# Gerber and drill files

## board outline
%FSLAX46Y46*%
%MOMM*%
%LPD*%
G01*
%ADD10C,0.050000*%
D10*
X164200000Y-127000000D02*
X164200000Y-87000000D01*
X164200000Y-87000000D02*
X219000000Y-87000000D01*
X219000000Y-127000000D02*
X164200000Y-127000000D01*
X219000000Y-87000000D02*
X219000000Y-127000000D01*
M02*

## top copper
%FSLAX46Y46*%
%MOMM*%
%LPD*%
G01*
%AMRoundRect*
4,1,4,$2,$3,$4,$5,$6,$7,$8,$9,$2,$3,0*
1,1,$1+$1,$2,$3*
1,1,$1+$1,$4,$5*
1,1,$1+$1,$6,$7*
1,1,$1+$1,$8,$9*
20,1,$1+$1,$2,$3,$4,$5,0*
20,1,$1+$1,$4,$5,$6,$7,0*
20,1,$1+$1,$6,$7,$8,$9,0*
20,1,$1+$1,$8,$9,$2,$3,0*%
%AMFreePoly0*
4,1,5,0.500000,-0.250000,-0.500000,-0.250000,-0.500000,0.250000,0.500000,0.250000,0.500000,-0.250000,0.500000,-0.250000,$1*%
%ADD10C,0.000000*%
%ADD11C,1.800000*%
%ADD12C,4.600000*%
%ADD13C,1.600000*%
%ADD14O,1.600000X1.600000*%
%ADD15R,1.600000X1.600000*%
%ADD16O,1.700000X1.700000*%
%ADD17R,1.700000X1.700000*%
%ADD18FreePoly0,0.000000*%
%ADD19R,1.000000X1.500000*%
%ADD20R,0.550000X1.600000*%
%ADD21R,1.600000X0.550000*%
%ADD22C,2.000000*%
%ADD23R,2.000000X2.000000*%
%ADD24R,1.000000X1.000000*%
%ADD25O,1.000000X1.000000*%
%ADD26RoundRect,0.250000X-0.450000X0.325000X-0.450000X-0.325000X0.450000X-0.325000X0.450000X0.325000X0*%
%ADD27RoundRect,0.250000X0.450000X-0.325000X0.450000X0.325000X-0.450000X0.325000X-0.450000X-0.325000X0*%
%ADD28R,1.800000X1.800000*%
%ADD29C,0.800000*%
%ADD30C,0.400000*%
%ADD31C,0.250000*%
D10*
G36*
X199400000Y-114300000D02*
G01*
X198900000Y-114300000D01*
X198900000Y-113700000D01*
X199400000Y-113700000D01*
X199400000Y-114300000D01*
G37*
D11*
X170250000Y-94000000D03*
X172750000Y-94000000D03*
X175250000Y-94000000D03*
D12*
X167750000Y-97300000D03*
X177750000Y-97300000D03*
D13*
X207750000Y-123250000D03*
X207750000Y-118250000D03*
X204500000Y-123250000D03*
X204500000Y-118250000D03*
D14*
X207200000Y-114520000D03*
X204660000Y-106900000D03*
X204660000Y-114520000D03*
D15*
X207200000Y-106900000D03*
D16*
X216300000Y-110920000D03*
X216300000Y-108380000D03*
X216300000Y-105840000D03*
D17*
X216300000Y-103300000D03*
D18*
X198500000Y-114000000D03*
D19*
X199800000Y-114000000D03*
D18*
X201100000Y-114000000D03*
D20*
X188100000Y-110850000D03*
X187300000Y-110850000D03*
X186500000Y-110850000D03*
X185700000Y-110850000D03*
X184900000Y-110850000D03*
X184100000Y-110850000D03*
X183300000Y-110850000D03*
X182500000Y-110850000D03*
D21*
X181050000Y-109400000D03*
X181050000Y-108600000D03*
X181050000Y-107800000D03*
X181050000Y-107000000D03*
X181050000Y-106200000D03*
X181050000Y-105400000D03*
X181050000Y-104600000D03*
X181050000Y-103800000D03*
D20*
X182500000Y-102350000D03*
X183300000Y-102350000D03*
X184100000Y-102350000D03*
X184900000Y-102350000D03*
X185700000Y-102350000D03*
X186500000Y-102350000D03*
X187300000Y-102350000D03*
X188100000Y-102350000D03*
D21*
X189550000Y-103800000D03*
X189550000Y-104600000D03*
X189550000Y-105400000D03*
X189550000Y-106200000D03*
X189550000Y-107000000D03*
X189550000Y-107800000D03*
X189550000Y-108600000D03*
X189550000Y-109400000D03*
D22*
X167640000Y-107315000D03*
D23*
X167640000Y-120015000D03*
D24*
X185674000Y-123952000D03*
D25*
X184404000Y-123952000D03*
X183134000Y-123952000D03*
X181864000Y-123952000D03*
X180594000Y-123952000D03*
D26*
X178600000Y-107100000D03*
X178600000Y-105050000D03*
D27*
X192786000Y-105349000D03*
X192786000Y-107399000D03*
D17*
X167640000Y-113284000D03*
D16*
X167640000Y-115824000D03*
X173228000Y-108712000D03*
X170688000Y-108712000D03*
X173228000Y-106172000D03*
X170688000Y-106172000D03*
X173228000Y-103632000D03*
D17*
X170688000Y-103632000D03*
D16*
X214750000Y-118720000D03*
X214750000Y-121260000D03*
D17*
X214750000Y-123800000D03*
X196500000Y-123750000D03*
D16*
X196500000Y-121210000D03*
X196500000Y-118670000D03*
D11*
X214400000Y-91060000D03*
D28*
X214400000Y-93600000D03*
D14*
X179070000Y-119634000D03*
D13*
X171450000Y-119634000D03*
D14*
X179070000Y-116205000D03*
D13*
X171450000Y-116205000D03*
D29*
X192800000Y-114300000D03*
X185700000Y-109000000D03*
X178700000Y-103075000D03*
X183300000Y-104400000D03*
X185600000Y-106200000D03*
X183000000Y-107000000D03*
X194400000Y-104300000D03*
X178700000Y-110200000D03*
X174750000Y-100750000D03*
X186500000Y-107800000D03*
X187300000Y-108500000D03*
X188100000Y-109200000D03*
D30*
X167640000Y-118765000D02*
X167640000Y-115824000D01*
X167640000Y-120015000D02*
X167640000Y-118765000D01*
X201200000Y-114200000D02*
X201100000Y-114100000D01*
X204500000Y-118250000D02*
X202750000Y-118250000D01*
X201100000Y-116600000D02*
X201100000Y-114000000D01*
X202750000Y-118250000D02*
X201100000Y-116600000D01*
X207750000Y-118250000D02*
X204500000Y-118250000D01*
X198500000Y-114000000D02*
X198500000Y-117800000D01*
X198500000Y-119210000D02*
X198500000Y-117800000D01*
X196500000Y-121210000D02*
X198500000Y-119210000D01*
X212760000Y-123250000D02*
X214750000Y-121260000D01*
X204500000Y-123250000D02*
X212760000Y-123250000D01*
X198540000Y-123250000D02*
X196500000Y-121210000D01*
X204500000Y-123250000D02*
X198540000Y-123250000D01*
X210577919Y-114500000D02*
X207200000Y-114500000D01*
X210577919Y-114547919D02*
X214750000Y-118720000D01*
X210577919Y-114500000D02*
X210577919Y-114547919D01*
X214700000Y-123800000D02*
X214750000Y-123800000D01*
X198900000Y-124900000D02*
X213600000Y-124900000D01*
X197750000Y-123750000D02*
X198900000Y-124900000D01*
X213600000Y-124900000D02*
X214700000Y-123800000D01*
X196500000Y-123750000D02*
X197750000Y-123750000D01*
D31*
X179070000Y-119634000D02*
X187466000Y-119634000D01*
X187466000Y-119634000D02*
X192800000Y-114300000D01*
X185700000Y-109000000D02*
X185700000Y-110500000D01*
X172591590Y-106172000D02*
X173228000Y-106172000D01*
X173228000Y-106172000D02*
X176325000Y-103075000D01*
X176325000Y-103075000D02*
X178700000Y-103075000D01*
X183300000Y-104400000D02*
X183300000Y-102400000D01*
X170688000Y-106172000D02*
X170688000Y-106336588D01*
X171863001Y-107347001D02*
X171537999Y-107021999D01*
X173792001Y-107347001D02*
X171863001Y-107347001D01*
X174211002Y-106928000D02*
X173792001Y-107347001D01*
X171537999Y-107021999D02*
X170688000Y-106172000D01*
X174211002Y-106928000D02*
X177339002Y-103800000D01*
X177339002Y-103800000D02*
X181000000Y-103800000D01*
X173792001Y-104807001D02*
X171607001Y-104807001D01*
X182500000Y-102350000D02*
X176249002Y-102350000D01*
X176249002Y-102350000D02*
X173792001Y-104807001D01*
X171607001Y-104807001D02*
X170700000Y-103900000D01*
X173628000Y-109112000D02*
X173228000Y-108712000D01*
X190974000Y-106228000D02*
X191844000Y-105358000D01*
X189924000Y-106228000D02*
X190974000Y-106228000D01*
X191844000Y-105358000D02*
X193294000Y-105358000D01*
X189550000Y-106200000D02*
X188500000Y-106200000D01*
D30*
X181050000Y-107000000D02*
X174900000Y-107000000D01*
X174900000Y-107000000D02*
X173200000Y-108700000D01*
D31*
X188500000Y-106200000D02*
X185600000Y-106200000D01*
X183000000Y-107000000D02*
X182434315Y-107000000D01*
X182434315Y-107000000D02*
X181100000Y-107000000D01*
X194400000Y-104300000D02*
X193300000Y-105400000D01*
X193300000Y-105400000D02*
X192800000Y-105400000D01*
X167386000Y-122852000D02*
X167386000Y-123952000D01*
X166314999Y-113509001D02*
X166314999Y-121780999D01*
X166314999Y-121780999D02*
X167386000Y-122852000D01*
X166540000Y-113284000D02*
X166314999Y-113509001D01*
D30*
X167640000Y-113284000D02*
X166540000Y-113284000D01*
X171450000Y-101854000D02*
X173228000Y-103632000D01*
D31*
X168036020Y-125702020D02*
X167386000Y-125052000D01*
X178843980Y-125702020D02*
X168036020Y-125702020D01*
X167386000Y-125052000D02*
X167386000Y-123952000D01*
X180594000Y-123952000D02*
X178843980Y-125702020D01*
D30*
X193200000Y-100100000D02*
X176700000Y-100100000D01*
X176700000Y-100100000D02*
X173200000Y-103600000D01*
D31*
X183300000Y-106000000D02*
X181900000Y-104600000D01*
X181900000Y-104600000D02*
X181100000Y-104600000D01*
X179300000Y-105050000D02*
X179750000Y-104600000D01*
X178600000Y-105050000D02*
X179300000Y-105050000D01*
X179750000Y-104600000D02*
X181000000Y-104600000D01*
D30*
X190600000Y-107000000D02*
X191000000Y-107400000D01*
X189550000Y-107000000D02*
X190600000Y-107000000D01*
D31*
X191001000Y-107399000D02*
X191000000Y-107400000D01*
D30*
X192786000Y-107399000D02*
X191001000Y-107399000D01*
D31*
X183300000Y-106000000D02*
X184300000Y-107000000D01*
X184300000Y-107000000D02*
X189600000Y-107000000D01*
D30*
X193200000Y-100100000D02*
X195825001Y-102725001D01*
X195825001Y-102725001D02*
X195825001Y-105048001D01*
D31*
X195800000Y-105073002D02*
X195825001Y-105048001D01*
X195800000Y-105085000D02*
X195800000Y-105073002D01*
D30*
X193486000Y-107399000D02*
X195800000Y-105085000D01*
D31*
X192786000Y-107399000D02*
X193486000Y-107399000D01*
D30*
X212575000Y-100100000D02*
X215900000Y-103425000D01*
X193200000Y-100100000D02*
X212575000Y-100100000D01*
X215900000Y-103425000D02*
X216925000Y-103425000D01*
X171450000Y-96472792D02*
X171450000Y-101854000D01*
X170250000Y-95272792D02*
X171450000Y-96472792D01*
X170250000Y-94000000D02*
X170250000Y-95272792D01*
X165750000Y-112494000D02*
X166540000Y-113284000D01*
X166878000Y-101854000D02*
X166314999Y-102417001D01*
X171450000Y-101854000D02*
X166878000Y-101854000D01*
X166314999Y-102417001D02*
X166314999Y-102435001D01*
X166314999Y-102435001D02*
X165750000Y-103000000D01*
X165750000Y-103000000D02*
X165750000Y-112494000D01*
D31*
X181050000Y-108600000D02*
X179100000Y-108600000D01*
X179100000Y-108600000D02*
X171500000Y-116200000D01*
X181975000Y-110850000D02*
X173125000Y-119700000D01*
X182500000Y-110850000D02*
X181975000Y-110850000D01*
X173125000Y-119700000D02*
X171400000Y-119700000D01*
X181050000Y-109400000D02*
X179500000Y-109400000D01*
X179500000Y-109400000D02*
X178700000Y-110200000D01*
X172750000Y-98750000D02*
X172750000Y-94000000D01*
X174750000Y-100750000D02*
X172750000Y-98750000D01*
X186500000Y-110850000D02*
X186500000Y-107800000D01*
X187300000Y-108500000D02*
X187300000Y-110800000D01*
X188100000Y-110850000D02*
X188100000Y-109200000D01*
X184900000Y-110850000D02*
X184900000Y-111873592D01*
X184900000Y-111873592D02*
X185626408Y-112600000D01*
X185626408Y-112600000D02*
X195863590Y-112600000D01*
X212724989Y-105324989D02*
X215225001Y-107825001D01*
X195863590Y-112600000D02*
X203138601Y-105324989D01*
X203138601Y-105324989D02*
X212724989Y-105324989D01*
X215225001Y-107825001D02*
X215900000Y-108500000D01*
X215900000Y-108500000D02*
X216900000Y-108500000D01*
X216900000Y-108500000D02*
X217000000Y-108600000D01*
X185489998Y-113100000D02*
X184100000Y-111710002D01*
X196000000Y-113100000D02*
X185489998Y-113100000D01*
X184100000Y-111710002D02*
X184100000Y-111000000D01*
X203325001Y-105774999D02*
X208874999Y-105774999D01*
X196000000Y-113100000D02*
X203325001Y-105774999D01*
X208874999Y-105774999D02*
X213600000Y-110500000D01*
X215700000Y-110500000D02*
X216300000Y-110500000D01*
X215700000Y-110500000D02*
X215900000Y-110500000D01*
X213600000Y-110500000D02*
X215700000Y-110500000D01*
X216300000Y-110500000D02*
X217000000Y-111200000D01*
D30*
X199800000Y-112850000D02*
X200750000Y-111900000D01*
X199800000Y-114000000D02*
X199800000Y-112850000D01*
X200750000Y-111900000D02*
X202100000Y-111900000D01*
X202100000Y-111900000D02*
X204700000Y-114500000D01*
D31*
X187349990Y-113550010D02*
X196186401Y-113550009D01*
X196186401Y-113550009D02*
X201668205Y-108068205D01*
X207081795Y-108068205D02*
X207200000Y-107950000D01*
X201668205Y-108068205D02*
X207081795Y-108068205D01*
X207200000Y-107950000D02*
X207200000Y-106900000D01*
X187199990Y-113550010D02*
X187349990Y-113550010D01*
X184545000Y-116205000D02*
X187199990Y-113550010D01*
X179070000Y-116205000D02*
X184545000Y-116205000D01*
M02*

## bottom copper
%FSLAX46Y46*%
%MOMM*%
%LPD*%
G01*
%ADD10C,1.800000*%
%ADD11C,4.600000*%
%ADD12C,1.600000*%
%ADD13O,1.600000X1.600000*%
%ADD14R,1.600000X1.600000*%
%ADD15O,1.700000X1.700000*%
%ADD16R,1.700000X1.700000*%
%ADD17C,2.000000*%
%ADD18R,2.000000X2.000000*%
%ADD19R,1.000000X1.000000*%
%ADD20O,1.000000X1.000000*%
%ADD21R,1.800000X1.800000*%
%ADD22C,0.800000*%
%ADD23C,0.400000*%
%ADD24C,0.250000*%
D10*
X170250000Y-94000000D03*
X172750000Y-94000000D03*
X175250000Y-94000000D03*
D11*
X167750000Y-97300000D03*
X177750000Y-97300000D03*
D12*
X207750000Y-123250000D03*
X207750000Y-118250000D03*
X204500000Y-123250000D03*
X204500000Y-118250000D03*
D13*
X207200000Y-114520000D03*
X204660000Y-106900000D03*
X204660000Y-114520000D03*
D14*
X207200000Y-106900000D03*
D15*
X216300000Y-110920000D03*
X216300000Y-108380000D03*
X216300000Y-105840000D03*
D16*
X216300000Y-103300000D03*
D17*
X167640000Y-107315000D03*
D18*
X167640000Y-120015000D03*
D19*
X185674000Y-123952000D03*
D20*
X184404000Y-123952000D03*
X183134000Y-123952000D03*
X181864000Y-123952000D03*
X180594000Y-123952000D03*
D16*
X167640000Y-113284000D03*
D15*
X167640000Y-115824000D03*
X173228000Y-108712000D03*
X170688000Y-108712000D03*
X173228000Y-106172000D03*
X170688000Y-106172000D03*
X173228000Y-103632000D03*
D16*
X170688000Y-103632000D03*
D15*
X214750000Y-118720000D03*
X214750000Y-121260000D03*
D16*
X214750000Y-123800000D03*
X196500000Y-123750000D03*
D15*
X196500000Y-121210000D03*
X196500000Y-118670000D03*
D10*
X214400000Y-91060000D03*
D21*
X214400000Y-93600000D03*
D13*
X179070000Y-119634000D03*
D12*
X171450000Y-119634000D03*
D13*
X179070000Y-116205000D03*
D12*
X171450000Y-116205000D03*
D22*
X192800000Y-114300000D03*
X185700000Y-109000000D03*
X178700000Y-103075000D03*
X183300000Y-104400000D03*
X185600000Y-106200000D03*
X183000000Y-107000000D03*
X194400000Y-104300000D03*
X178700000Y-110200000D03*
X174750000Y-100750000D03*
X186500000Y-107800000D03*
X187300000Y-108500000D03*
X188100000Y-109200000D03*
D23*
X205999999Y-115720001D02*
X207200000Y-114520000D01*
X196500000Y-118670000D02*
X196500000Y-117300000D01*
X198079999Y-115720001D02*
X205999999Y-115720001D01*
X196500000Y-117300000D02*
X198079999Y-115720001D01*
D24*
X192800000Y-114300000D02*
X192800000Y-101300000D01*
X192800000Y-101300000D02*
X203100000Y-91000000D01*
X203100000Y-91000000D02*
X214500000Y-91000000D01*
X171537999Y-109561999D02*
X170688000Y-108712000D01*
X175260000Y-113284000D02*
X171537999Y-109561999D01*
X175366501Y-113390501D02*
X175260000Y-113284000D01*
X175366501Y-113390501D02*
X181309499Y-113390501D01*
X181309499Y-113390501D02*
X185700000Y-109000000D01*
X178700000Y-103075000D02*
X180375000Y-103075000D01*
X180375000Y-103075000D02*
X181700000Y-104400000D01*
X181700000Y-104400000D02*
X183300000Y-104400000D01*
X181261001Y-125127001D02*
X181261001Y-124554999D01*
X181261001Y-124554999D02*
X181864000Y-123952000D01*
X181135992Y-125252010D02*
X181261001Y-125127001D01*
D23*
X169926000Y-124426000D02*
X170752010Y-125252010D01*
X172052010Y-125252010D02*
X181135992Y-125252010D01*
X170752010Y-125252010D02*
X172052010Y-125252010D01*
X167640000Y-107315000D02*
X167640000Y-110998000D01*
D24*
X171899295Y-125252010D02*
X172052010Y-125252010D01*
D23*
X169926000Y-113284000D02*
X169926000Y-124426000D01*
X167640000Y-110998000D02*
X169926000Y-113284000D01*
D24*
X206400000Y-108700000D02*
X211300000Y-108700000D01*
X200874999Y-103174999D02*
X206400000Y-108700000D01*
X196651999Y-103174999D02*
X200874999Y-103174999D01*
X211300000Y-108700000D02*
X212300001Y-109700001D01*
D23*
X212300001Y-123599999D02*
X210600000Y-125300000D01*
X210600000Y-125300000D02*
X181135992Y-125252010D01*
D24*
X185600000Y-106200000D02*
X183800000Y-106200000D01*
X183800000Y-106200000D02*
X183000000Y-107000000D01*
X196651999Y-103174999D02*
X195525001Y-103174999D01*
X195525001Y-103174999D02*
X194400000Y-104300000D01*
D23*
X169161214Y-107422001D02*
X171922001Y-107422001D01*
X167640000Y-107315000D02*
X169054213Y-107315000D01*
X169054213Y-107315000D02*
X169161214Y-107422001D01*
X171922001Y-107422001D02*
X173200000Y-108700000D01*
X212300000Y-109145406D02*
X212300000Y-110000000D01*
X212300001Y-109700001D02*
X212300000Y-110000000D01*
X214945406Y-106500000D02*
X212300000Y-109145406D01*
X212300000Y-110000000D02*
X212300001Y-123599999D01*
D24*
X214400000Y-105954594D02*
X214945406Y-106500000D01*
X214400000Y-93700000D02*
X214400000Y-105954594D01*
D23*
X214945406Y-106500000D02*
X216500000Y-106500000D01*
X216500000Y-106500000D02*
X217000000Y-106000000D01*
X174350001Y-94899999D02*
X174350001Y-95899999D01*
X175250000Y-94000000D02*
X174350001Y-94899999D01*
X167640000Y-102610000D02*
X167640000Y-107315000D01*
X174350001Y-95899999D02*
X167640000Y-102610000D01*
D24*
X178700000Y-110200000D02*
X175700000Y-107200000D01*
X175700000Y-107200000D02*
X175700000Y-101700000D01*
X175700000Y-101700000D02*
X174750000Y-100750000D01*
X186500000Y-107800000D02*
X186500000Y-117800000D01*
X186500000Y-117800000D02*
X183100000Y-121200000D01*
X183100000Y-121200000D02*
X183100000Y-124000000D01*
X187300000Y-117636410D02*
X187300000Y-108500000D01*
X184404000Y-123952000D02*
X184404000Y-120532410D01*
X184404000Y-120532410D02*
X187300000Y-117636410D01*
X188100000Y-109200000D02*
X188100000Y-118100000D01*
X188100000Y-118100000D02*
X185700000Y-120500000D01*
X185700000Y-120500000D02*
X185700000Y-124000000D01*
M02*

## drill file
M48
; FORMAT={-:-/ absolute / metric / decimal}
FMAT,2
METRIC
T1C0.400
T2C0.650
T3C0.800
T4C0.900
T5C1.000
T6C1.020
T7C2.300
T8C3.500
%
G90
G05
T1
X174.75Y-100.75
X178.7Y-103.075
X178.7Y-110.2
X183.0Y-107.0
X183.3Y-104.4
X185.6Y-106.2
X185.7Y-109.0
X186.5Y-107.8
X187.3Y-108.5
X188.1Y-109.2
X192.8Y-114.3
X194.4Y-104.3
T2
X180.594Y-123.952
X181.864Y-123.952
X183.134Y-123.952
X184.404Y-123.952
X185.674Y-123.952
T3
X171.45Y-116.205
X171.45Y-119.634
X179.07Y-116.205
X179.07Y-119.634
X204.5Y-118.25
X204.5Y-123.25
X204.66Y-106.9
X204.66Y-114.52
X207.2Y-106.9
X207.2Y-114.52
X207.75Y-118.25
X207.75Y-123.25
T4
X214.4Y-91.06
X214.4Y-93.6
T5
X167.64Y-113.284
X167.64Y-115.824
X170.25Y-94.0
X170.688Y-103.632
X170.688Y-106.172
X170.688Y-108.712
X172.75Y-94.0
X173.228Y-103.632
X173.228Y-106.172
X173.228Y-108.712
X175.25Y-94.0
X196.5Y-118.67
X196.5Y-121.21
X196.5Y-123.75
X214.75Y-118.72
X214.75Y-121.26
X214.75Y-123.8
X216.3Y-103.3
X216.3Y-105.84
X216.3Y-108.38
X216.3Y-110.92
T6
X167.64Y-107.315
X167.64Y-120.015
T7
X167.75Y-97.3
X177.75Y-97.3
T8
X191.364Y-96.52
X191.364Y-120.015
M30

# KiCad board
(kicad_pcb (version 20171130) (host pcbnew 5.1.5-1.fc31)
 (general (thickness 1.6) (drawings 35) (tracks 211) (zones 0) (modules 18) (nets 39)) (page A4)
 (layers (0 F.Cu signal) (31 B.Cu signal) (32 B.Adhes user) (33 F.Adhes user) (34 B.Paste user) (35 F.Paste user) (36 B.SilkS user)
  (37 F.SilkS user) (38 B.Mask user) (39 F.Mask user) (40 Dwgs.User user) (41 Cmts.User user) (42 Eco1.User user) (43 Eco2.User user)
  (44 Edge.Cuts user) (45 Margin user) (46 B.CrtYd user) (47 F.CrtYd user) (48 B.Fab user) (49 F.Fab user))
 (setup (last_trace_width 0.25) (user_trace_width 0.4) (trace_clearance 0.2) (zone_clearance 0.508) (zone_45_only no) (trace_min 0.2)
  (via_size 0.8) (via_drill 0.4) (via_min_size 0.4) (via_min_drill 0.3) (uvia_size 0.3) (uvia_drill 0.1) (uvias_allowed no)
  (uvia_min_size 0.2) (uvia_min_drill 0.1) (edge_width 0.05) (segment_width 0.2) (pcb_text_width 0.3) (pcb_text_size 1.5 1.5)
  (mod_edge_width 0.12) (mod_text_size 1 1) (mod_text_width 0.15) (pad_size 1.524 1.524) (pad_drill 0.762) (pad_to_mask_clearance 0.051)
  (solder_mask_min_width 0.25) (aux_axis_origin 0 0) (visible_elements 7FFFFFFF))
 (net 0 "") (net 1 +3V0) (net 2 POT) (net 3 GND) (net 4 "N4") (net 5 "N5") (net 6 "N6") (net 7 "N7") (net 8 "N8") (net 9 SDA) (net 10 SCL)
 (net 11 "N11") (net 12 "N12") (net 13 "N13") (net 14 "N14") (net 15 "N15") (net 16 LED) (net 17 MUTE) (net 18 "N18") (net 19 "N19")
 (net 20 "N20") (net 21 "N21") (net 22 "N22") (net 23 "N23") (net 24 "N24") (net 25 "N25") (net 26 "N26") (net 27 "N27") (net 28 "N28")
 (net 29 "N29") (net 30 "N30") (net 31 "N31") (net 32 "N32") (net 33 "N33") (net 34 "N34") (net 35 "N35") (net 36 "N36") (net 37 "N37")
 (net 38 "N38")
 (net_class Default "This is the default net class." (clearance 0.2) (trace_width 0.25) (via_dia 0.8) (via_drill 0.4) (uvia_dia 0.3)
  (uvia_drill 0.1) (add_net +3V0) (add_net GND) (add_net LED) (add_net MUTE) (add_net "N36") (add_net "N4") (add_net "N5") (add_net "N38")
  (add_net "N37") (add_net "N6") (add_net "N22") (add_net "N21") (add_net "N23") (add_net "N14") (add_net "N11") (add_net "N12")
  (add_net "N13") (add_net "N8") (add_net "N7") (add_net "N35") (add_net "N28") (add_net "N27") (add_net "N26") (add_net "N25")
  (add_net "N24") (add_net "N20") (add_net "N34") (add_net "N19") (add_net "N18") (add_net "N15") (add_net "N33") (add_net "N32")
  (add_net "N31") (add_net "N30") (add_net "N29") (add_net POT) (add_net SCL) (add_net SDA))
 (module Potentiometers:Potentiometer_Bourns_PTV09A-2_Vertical (layer F.Cu) (at 175.25 94 90)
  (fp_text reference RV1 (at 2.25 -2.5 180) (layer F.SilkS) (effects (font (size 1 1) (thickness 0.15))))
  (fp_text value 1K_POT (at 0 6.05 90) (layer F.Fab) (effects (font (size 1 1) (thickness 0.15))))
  (pad 3 thru_hole circle (at 0 -5 90) (size 1.8 1.8) (drill 1) (layers *.Cu *.Mask) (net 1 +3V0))
  (pad 2 thru_hole circle (at 0 -2.5 90) (size 1.8 1.8) (drill 1) (layers *.Cu *.Mask) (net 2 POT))
  (pad 1 thru_hole circle (at 0 0 90) (size 1.8 1.8) (drill 1) (layers *.Cu *.Mask) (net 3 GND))
  (pad 0 thru_hole circle (at -3.3 -7.5 90) (size 4.6 4.6) (drill 2.3) (layers *.Cu *.Mask))
  (pad 0 thru_hole circle (at -3.3 2.5 90) (size 4.6 4.6) (drill 2.3) (layers *.Cu *.Mask)))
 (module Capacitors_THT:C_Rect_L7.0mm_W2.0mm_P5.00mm (layer F.Cu) (at 207.75 123.25 90)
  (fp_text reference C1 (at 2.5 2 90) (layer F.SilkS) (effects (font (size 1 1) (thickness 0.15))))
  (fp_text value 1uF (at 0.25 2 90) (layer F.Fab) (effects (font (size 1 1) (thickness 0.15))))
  (pad 1 thru_hole circle (at 0 0 90) (size 1.6 1.6) (drill 0.8) (layers *.Cu *.Mask) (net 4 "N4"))
  (pad 2 thru_hole circle (at 5 0 90) (size 1.6 1.6) (drill 0.8) (layers *.Cu *.Mask) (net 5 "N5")))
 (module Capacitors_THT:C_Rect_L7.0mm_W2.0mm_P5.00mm (layer F.Cu) (at 204.5 123.25 90)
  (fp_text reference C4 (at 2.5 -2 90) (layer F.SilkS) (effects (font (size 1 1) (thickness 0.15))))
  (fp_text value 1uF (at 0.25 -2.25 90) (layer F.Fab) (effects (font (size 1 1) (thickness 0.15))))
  (pad 1 thru_hole circle (at 0 0 90) (size 1.6 1.6) (drill 0.8) (layers *.Cu *.Mask) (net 4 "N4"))
  (pad 2 thru_hole circle (at 5 0 90) (size 1.6 1.6) (drill 0.8) (layers *.Cu *.Mask) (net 5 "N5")))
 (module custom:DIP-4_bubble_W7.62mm (layer F.Cu) (at 207.2 106.9 270)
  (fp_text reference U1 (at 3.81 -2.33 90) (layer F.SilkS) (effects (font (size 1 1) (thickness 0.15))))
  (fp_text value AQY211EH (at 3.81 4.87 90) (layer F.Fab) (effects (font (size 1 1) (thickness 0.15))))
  (pad 4 thru_hole oval (at 7.62 0 270) (size 1.6 1.6) (drill 0.8) (layers *.Cu *.Mask) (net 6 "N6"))
  (pad 2 thru_hole oval (at 0 2.54 270) (size 1.6 1.6) (drill 0.8) (layers *.Cu *.Mask) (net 3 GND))
  (pad 3 thru_hole oval (at 7.62 2.54 270) (size 1.6 1.6) (drill 0.8) (layers *.Cu *.Mask) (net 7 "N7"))
  (pad 1 thru_hole rect (at 0 0 270) (size 1.6 1.6) (drill 0.8) (layers *.Cu *.Mask) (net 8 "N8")))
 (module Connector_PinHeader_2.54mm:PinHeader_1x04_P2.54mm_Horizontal (layer F.Cu) (at 216.3 103.3)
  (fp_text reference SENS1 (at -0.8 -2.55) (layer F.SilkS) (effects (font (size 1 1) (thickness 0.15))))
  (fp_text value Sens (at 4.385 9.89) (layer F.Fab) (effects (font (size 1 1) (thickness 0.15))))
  (pad 4 thru_hole oval (at 0 7.62) (size 1.7 1.7) (drill 1) (layers *.Cu *.Mask) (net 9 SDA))
  (pad 3 thru_hole oval (at 0 5.08) (size 1.7 1.7) (drill 1) (layers *.Cu *.Mask) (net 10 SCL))
  (pad 2 thru_hole oval (at 0 2.54) (size 1.7 1.7) (drill 1) (layers *.Cu *.Mask) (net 3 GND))
  (pad 1 thru_hole rect (at 0 0) (size 1.7 1.7) (drill 1) (layers *.Cu *.Mask) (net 1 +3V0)))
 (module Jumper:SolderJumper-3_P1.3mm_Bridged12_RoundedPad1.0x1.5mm (layer F.Cu) (at 199.8 114)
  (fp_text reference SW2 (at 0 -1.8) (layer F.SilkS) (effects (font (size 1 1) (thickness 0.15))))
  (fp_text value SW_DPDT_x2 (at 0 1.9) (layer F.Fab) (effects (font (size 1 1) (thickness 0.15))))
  (fp_poly (pts (xy -0.9 -0.3) (xy -0.4 -0.3) (xy -0.4 0.3) (xy -0.9 0.3)) (layer F.Cu) (width 0))
  (pad 1 smd custom (at -1.3 0) (size 1 0.5) (layers F.Cu F.Mask) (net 4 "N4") (zone_connect 2) (options (clearance outline) (anchor rect))
   (primitives))
  (pad 2 smd rect (at 0 0) (size 1 1.5) (layers F.Cu F.Mask) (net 7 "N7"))
  (pad 3 smd custom (at 1.3 0) (size 1 0.5) (layers F.Cu F.Mask) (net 5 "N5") (zone_connect 2) (options (clearance outline) (anchor rect))
   (primitives)))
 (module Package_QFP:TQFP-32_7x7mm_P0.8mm (layer F.Cu) (at 185.3 106.6 180)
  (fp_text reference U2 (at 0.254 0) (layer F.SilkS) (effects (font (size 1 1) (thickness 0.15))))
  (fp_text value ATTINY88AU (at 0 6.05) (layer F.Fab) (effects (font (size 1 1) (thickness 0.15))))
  (pad 32 smd rect (at -2.8 -4.25 270) (size 1.6 0.55) (layers F.Cu F.Paste F.Mask) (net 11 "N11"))
  (pad 31 smd rect (at -2 -4.25 270) (size 1.6 0.55) (layers F.Cu F.Paste F.Mask) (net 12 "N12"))
  (pad 30 smd rect (at -1.2 -4.25 270) (size 1.6 0.55) (layers F.Cu F.Paste F.Mask) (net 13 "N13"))
  (pad 29 smd rect (at -0.4 -4.25 270) (size 1.6 0.55) (layers F.Cu F.Paste F.Mask) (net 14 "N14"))
  (pad 28 smd rect (at 0.4 -4.25 270) (size 1.6 0.55) (layers F.Cu F.Paste F.Mask) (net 10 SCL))
  (pad 27 smd rect (at 1.2 -4.25 270) (size 1.6 0.55) (layers F.Cu F.Paste F.Mask) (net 9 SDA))
  (pad 26 smd rect (at 2 -4.25 270) (size 1.6 0.55) (layers F.Cu F.Paste F.Mask) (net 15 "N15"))
  (pad 25 smd rect (at 2.8 -4.25 270) (size 1.6 0.55) (layers F.Cu F.Paste F.Mask) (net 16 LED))
  (pad 24 smd rect (at 4.25 -2.8 180) (size 1.6 0.55) (layers F.Cu F.Paste F.Mask) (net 2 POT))
  (pad 23 smd rect (at 4.25 -2 180) (size 1.6 0.55) (layers F.Cu F.Paste F.Mask) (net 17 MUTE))
  (pad 22 smd rect (at 4.25 -1.2 180) (size 1.6 0.55) (layers F.Cu F.Paste F.Mask) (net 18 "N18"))
  (pad 21 smd rect (at 4.25 -0.4 180) (size 1.6 0.55) (layers F.Cu F.Paste F.Mask) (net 3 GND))
  (pad 20 smd rect (at 4.25 0.4 180) (size 1.6 0.55) (layers F.Cu F.Paste F.Mask) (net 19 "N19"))
  (pad 19 smd rect (at 4.25 1.2 180) (size 1.6 0.55) (layers F.Cu F.Paste F.Mask) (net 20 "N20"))
  (pad 18 smd rect (at 4.25 2 180) (size 1.6 0.55) (layers F.Cu F.Paste F.Mask) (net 1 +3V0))
  (pad 17 smd rect (at 4.25 2.8 180) (size 1.6 0.55) (layers F.Cu F.Paste F.Mask) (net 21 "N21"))
  (pad 16 smd rect (at 2.8 4.25 270) (size 1.6 0.55) (layers F.Cu F.Paste F.Mask) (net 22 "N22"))
  (pad 15 smd rect (at 2 4.25 270) (size 1.6 0.55) (layers F.Cu F.Paste F.Mask) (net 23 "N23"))
  (pad 14 smd rect (at 1.2 4.25 270) (size 1.6 0.55) (layers F.Cu F.Paste F.Mask) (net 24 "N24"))
  (pad 13 smd rect (at 0.4 4.25 270) (size 1.6 0.55) (layers F.Cu F.Paste F.Mask) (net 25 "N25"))
  (pad 12 smd rect (at -0.4 4.25 270) (size 1.6 0.55) (layers F.Cu F.Paste F.Mask) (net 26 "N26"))
  (pad 11 smd rect (at -1.2 4.25 270) (size 1.6 0.55) (layers F.Cu F.Paste F.Mask) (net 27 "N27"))
  (pad 10 smd rect (at -2 4.25 270) (size 1.6 0.55) (layers F.Cu F.Paste F.Mask) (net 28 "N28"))
  (pad 9 smd rect (at -2.8 4.25 270) (size 1.6 0.55) (layers F.Cu F.Paste F.Mask) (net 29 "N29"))
  (pad 8 smd rect (at -4.25 2.8 180) (size 1.6 0.55) (layers F.Cu F.Paste F.Mask) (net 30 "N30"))
  (pad 7 smd rect (at -4.25 2 180) (size 1.6 0.55) (layers F.Cu F.Paste F.Mask) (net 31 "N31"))
  (pad 6 smd rect (at -4.25 1.2 180) (size 1.6 0.55) (layers F.Cu F.Paste F.Mask) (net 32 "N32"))
  (pad 5 smd rect (at -4.25 0.4 180) (size 1.6 0.55) (layers F.Cu F.Paste F.Mask) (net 3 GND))
  (pad 4 smd rect (at -4.25 -0.4 180) (size 1.6 0.55) (layers F.Cu F.Paste F.Mask) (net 1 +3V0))
  (pad 3 smd rect (at -4.25 -1.2 180) (size 1.6 0.55) (layers F.Cu F.Paste F.Mask) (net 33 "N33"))
  (pad 2 smd rect (at -4.25 -2 180) (size 1.6 0.55) (layers F.Cu F.Paste F.Mask) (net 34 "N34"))
  (pad 1 smd rect (at -4.25 -2.8 180) (size 1.6 0.55) (layers F.Cu F.Paste F.Mask) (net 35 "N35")))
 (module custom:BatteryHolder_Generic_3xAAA (layer B.Cu) (at 167.64 120.015)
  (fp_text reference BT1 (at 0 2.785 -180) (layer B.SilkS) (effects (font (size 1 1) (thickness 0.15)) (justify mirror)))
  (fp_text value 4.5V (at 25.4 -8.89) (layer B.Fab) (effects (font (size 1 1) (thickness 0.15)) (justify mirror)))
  (pad "" np_thru_hole circle (at 23.7236 0) (size 3.5 3.5) (drill 3.5) (layers *.Cu *.Mask))
  (pad "" np_thru_hole circle (at 23.7236 -23.495) (size 3.5 3.5) (drill 3.5) (layers *.Cu *.Mask))
  (pad 2 thru_hole circle (at 0 -12.7) (size 2 2) (drill 1.02) (layers *.Cu *.Mask) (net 3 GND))
  (pad 1 thru_hole rect (at 0 0) (size 2 2) (drill 1.02) (layers *.Cu *.Mask) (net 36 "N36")))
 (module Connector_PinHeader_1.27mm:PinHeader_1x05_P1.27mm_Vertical (layer F.Cu) (at 185.674 123.952 270)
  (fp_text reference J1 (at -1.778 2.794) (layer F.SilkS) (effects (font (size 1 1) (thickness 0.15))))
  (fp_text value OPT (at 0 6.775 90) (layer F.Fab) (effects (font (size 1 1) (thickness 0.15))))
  (pad 1 thru_hole rect (at 0 0 270) (size 1 1) (drill 0.65) (layers *.Cu *.Mask) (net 11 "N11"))
  (pad 2 thru_hole oval (at 0 1.27 270) (size 1 1) (drill 0.65) (layers *.Cu *.Mask) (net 12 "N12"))
  (pad 3 thru_hole oval (at 0 2.54 270) (size 1 1) (drill 0.65) (layers *.Cu *.Mask) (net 13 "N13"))
  (pad 4 thru_hole oval (at 0 3.81 270) (size 1 1) (drill 0.65) (layers *.Cu *.Mask) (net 3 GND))
  (pad 5 thru_hole oval (at 0 5.08 270) (size 1 1) (drill 0.65) (layers *.Cu *.Mask) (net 1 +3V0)))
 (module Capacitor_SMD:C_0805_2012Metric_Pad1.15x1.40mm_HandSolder (layer F.Cu) (at 178.6 106.075 270)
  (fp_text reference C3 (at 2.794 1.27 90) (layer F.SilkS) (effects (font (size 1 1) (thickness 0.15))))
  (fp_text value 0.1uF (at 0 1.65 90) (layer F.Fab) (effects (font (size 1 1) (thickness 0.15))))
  (pad 2 smd roundrect (at 1.025 0 270) (size 1.15 1.4) (layers F.Cu F.Paste F.Mask) (roundrect_rratio 0.217391) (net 3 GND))
  (pad 1 smd roundrect (at -1.025 0 270) (size 1.15 1.4) (layers F.Cu F.Paste F.Mask) (roundrect_rratio 0.217391) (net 1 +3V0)))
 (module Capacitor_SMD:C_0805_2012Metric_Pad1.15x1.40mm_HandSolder (layer F.Cu) (at 192.786 106.374 90)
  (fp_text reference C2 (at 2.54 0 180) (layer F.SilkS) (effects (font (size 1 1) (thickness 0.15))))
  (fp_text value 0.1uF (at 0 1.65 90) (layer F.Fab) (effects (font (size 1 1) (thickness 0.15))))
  (pad 2 smd roundrect (at 1.025 0 90) (size 1.15 1.4) (layers F.Cu F.Paste F.Mask) (roundrect_rratio 0.217391) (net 3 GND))
  (pad 1 smd roundrect (at -1.025 0 90) (size 1.15 1.4) (layers F.Cu F.Paste F.Mask) (roundrect_rratio 0.217391) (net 1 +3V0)))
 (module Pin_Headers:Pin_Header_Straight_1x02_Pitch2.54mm (layer F.Cu) (at 167.64 113.284)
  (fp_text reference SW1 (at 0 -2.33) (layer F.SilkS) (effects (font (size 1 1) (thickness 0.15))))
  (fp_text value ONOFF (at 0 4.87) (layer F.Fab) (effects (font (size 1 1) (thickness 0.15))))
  (pad 1 thru_hole rect (at 0 0) (size 1.7 1.7) (drill 1) (layers *.Cu *.Mask) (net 1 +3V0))
  (pad 2 thru_hole oval (at 0 2.54) (size 1.7 1.7) (drill 1) (layers *.Cu *.Mask) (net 36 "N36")))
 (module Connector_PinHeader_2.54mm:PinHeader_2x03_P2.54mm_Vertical (layer F.Cu) (at 170.688 103.632)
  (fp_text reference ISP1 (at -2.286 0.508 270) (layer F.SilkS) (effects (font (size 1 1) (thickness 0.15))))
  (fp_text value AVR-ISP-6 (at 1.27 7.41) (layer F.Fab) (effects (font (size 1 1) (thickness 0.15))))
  (pad 6 thru_hole oval (at 2.54 5.08) (size 1.7 1.7) (drill 1) (layers *.Cu *.Mask) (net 3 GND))
  (pad 5 thru_hole oval (at 0 5.08) (size 1.7 1.7) (drill 1) (layers *.Cu *.Mask) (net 14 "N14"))
  (pad 4 thru_hole oval (at 2.54 2.54) (size 1.7 1.7) (drill 1) (layers *.Cu *.Mask) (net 23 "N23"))
  (pad 3 thru_hole oval (at 0 2.54) (size 1.7 1.7) (drill 1) (layers *.Cu *.Mask) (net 21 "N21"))
  (pad 2 thru_hole oval (at 2.54 0) (size 1.7 1.7) (drill 1) (layers *.Cu *.Mask) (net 1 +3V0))
  (pad 1 thru_hole rect (at 0 0) (size 1.7 1.7) (drill 1) (layers *.Cu *.Mask) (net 22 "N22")))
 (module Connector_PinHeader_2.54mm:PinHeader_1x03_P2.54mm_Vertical (layer F.Cu) (at 214.75 123.8 180)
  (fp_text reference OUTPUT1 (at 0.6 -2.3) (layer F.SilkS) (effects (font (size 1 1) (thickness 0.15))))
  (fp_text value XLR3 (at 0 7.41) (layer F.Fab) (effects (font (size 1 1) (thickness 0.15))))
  (pad 3 thru_hole oval (at 0 5.08 180) (size 1.7 1.7) (drill 1) (layers *.Cu *.Mask) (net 6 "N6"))
  (pad 2 thru_hole oval (at 0 2.54 180) (size 1.7 1.7) (drill 1) (layers *.Cu *.Mask) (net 4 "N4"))
  (pad 1 thru_hole rect (at 0 0 180) (size 1.7 1.7) (drill 1) (layers *.Cu *.Mask) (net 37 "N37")))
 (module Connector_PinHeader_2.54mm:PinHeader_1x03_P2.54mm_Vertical (layer F.Cu) (at 196.5 123.75 180)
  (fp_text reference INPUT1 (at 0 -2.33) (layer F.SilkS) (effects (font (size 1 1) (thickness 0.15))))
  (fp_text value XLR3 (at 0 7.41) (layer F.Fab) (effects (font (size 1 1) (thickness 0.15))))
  (pad 1 thru_hole rect (at 0 0 180) (size 1.7 1.7) (drill 1) (layers *.Cu *.Mask) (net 37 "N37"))
  (pad 2 thru_hole oval (at 0 2.54 180) (size 1.7 1.7) (drill 1) (layers *.Cu *.Mask) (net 4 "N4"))
  (pad 3 thru_hole oval (at 0 5.08 180) (size 1.7 1.7) (drill 1) (layers *.Cu *.Mask) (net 6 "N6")))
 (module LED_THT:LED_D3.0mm (layer F.Cu) (at 214.4 93.6 90)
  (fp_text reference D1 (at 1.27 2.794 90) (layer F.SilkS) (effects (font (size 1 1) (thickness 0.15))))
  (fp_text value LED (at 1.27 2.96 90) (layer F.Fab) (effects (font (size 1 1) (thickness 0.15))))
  (pad 2 thru_hole circle (at 2.54 0 90) (size 1.8 1.8) (drill 0.9) (layers *.Cu *.Mask) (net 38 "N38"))
  (pad 1 thru_hole rect (at 0 0 90) (size 1.8 1.8) (drill 0.9) (layers *.Cu *.Mask) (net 3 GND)))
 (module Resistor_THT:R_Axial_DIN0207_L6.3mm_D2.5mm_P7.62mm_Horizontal (layer F.Cu) (at 171.45 119.634)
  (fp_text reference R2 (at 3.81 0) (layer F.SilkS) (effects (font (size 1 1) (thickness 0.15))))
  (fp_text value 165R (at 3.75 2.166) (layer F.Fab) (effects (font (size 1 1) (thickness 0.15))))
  (pad 2 thru_hole oval (at 7.62 0) (size 1.6 1.6) (drill 0.8) (layers *.Cu *.Mask) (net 38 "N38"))
  (pad 1 thru_hole circle (at 0 0) (size 1.6 1.6) (drill 0.8) (layers *.Cu *.Mask) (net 16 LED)))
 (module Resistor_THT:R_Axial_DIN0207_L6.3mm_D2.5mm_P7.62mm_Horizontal (layer F.Cu) (at 171.45 116.205)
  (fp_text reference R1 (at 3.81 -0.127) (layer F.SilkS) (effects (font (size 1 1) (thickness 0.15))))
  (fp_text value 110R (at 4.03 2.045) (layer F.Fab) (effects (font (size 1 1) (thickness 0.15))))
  (pad 2 thru_hole oval (at 7.62 0) (size 1.6 1.6) (drill 0.8) (layers *.Cu *.Mask) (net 8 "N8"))
  (pad 1 thru_hole circle (at 0 0) (size 1.6 1.6) (drill 0.8) (layers *.Cu *.Mask) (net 17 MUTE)))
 (gr_line (start 164.2 127) (end 164.2 87) (layer Edge.Cuts) (width 0.05))
 (gr_line (start 164.2 87) (end 219 87) (layer Edge.Cuts) (width 0.05))
 (gr_line (start 219 127) (end 164.2 127) (layer Edge.Cuts) (width 0.05))
 (gr_line (start 219 87) (end 219 127) (layer Edge.Cuts) (width 0.05))
 (segment (start 167.64 118.765) (end 167.64 115.824) (width 0.4) (layer F.Cu) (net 36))
 (segment (start 167.64 120.015) (end 167.64 118.765) (width 0.4) (layer F.Cu) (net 36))
 (segment (start 201.2 114.2) (end 201.1 114.1) (width 0.4) (layer F.Cu) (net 5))
 (segment (start 204.5 118.25) (end 202.75 118.25) (width 0.4) (layer F.Cu) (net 5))
 (segment (start 201.1 116.6) (end 201.1 114) (width 0.4) (layer F.Cu) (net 5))
 (segment (start 202.75 118.25) (end 201.1 116.6) (width 0.4) (layer F.Cu) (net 5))
 (segment (start 207.75 118.25) (end 204.5 118.25) (width 0.4) (layer F.Cu) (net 5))
 (segment (start 198.5 114) (end 198.5 117.8) (width 0.4) (layer F.Cu) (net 4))
 (segment (start 198.5 119.21) (end 198.5 117.8) (width 0.4) (layer F.Cu) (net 4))
 (segment (start 196.5 121.21) (end 198.5 119.21) (width 0.4) (layer F.Cu) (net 4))
 (segment (start 212.76 123.25) (end 214.75 121.26) (width 0.4) (layer F.Cu) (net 4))
 (segment (start 204.5 123.25) (end 212.76 123.25) (width 0.4) (layer F.Cu) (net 4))
 (segment (start 198.54 123.25) (end 196.5 121.21) (width 0.4) (layer F.Cu) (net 4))
 (segment (start 204.5 123.25) (end 198.54 123.25) (width 0.4) (layer F.Cu) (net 4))
 (segment (start 210.577919 114.5) (end 207.2 114.5) (width 0.4) (layer F.Cu) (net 6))
 (segment (start 205.999999 115.720001) (end 207.2 114.52) (width 0.4) (layer B.Cu) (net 6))
 (segment (start 196.5 118.67) (end 196.5 117.3) (width 0.4) (layer B.Cu) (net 6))
 (segment (start 198.079999 115.720001) (end 205.999999 115.720001) (width 0.4) (layer B.Cu) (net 6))
 (segment (start 196.5 117.3) (end 198.079999 115.720001) (width 0.4) (layer B.Cu) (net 6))
 (segment (start 210.577919 114.547919) (end 214.75 118.72) (width 0.4) (layer F.Cu) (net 6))
 (segment (start 210.577919 114.5) (end 210.577919 114.547919) (width 0.4) (layer F.Cu) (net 6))
 (segment (start 214.7 123.8) (end 214.75 123.8) (width 0.4) (layer F.Cu) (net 37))
 (segment (start 198.9 124.9) (end 213.6 124.9) (width 0.4) (layer F.Cu) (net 37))
 (segment (start 197.75 123.75) (end 198.9 124.9) (width 0.4) (layer F.Cu) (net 37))
 (segment (start 213.6 124.9) (end 214.7 123.8) (width 0.4) (layer F.Cu) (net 37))
 (segment (start 196.5 123.75) (end 197.75 123.75) (width 0.4) (layer F.Cu) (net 37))
 (via (at 192.8 114.3) (size 0.8) (drill 0.4) (layers F.Cu B.Cu) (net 38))
 (segment (start 179.07 119.634) (end 187.466 119.634) (width 0.25) (layer F.Cu) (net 38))
 (segment (start 187.466 119.634) (end 192.8 114.3) (width 0.25) (layer F.Cu) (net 38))
 (segment (start 192.8 114.3) (end 192.8 101.3) (width 0.25) (layer B.Cu) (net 38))
 (segment (start 192.8 101.3) (end 203.1 91) (width 0.25) (layer B.Cu) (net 38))
 (segment (start 203.1 91) (end 214.5 91) (width 0.25) (layer B.Cu) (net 38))
 (segment (start 171.537999 109.561999) (end 170.688 108.712) (width 0.25) (layer B.Cu) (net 14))
 (segment (start 175.26 113.284) (end 171.537999 109.561999) (width 0.25) (layer B.Cu) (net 14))
 (segment (start 175.366501 113.390501) (end 175.26 113.284) (width 0.25) (layer B.Cu) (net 14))
 (via (at 185.7 109) (size 0.8) (drill 0.4) (layers F.Cu B.Cu) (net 14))
 (segment (start 175.366501 113.390501) (end 181.309499 113.390501) (width 0.25) (layer B.Cu) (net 14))
 (segment (start 181.309499 113.390501) (end 185.7 109) (width 0.25) (layer B.Cu) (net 14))
 (segment (start 185.7 109) (end 185.7 110.5) (width 0.25) (layer F.Cu) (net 14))
 (segment (start 172.59159 106.172) (end 173.228 106.172) (width 0.25) (layer F.Cu) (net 23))
 (via (at 178.7 103.075) (size 0.8) (drill 0.4) (layers F.Cu B.Cu) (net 23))
 (segment (start 173.228 106.172) (end 176.325 103.075) (width 0.25) (layer F.Cu) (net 23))
 (segment (start 176.325 103.075) (end 178.7 103.075) (width 0.25) (layer F.Cu) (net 23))
 (segment (start 178.7 103.075) (end 180.375 103.075) (width 0.25) (layer B.Cu) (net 23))
 (via (at 183.3 104.4) (size 0.8) (drill 0.4) (layers F.Cu B.Cu) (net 23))
 (segment (start 180.375 103.075) (end 181.7 104.4) (width 0.25) (layer B.Cu) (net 23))
 (segment (start 181.7 104.4) (end 183.3 104.4) (width 0.25) (layer B.Cu) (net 23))
 (segment (start 183.3 104.4) (end 183.3 102.4) (width 0.25) (layer F.Cu) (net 23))
 (segment (start 170.688 106.172) (end 170.688 106.336588) (width 0.25) (layer F.Cu) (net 21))
 (segment (start 171.863001 107.347001) (end 171.537999 107.021999) (width 0.25) (layer F.Cu) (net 21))
 (segment (start 173.792001 107.347001) (end 171.863001 107.347001) (width 0.25) (layer F.Cu) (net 21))
 (segment (start 174.211002 106.928) (end 173.792001 107.347001) (width 0.25) (layer F.Cu) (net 21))
 (segment (start 171.537999 107.021999) (end 170.688 106.172) (width 0.25) (layer F.Cu) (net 21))
 (segment (start 174.211002 106.928) (end 177.339002 103.8) (width 0.25) (layer F.Cu) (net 21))
 (segment (start 177.339002 103.8) (end 181 103.8) (width 0.25) (layer F.Cu) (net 21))
 (segment (start 173.792001 104.807001) (end 171.607001 104.807001) (width 0.25) (layer F.Cu) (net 22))
 (segment (start 182.5 102.35) (end 176.249002 102.35) (width 0.25) (layer F.Cu) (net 22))
 (segment (start 176.249002 102.35) (end 173.792001 104.807001) (width 0.25) (layer F.Cu) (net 22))
 (segment (start 171.607001 104.807001) (end 170.7 103.9) (width 0.25) (layer F.Cu) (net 22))
 (segment (start 173.628 109.112) (end 173.228 108.712) (width 0.25) (layer F.Cu) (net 3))
 (segment (start 190.974 106.228) (end 191.844 105.358) (width 0.25) (layer F.Cu) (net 3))
 (segment (start 189.924 106.228) (end 190.974 106.228) (width 0.25) (layer F.Cu) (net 3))
 (segment (start 191.844 105.358) (end 193.294 105.358) (width 0.25) (layer F.Cu) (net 3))
 (segment (start 181.261001 125.127001) (end 181.261001 124.554999) (width 0.25) (layer B.Cu) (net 3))
 (segment (start 181.261001 124.554999) (end 181.864 123.952) (width 0.25) (layer B.Cu) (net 3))
 (segment (start 181.135992 125.25201) (end 181.261001 125.127001) (width 0.25) (layer B.Cu) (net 3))
 (segment (start 189.55 106.2) (end 188.5 106.2) (width 0.25) (layer F.Cu) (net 3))
 (segment (start 181.05 107) (end 174.9 107) (width 0.4) (layer F.Cu) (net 3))
 (segment (start 174.9 107) (end 173.2 108.7) (width 0.4) (layer F.Cu) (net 3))
 (segment (start 169.926 124.426) (end 170.75201 125.25201) (width 0.4) (layer B.Cu) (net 3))
 (segment (start 172.05201 125.25201) (end 181.135992 125.25201) (width 0.4) (layer B.Cu) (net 3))
 (segment (start 170.75201 125.25201) (end 172.05201 125.25201) (width 0.4) (layer B.Cu) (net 3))
 (segment (start 167.64 107.315) (end 167.64 110.998) (width 0.4) (layer B.Cu) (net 3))
 (segment (start 171.899295 125.25201) (end 172.05201 125.25201) (width 0.25) (layer B.Cu) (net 3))
 (segment (start 169.926 113.284) (end 169.926 124.426) (width 0.4) (layer B.Cu) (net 3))
 (segment (start 167.64 110.998) (end 169.926 113.284) (width 0.4) (layer B.Cu) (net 3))
 (segment (start 206.4 108.7) (end 211.3 108.7) (width 0.25) (layer B.Cu) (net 3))
 (segment (start 200.874999 103.174999) (end 206.4 108.7) (width 0.25) (layer B.Cu) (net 3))
 (segment (start 196.651999 103.174999) (end 200.874999 103.174999) (width 0.25) (layer B.Cu) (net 3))
 (segment (start 211.3 108.7) (end 212.300001 109.700001) (width 0.25) (layer B.Cu) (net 3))
 (segment (start 212.300001 123.599999) (end 210.6 125.3) (width 0.4) (layer B.Cu) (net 3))
 (segment (start 210.6 125.3) (end 181.135992 125.25201) (width 0.4) (layer B.Cu) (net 3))
 (via (at 185.6 106.2) (size 0.8) (drill 0.4) (layers F.Cu B.Cu) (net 3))
 (segment (start 188.5 106.2) (end 185.6 106.2) (width 0.25) (layer F.Cu) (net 3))
 (via (at 183 107) (size 0.8) (drill 0.4) (layers F.Cu B.Cu) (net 3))
 (segment (start 185.6 106.2) (end 183.8 106.2) (width 0.25) (layer B.Cu) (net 3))
 (segment (start 183.8 106.2) (end 183 107) (width 0.25) (layer B.Cu) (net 3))
 (segment (start 183 107) (end 182.434315 107) (width 0.25) (layer F.Cu) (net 3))
 (segment (start 182.434315 107) (end 181.1 107) (width 0.25) (layer F.Cu) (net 3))
 (segment (start 196.651999 103.174999) (end 195.525001 103.174999) (width 0.25) (layer B.Cu) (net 3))
 (via (at 194.4 104.3) (size 0.8) (drill 0.4) (layers F.Cu B.Cu) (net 3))
 (segment (start 195.525001 103.174999) (end 194.4 104.3) (width 0.25) (layer B.Cu) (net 3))
 (segment (start 194.4 104.3) (end 193.3 105.4) (width 0.25) (layer F.Cu) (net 3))
 (segment (start 193.3 105.4) (end 192.8 105.4) (width 0.25) (layer F.Cu) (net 3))
 (segment (start 169.161214 107.422001) (end 171.922001 107.422001) (width 0.4) (layer B.Cu) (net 3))
 (segment (start 167.64 107.315) (end 169.054213 107.315) (width 0.4) (layer B.Cu) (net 3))
 (segment (start 169.054213 107.315) (end 169.161214 107.422001) (width 0.4) (layer B.Cu) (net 3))
 (segment (start 171.922001 107.422001) (end 173.2 108.7) (width 0.4) (layer B.Cu) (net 3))
 (segment (start 212.3 109.145406) (end 212.3 110) (width 0.4) (layer B.Cu) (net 3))
 (segment (start 212.300001 109.700001) (end 212.3 110) (width 0.4) (layer B.Cu) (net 3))
 (segment (start 214.945406 106.5) (end 212.3 109.145406) (width 0.4) (layer B.Cu) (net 3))
 (segment (start 212.3 110) (end 212.300001 123.599999) (width 0.4) (layer B.Cu) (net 3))
 (segment (start 214.4 105.954594) (end 214.945406 106.5) (width 0.25) (layer B.Cu) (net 3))
 (segment (start 214.4 93.7) (end 214.4 105.954594) (width 0.25) (layer B.Cu) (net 3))
 (segment (start 214.945406 106.5) (end 216.5 106.5) (width 0.4) (layer B.Cu) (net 3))
 (segment (start 216.5 106.5) (end 217 106) (width 0.4) (layer B.Cu) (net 3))
 (segment (start 174.350001 94.899999) (end 174.350001 95.899999) (width 0.4) (layer B.Cu) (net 3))
 (segment (start 175.25 94) (end 174.350001 94.899999) (width 0.4) (layer B.Cu) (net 3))
 (segment (start 167.64 102.61) (end 167.64 107.315) (width 0.4) (layer B.Cu) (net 3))
 (segment (start 174.350001 95.899999) (end 167.64 102.61) (width 0.4) (layer B.Cu) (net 3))
 (segment (start 167.386 122.852) (end 167.386 123.952) (width 0.25) (layer F.Cu) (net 1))
 (segment (start 166.314999 113.509001) (end 166.314999 121.780999) (width 0.25) (layer F.Cu) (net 1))
 (segment (start 166.314999 121.780999) (end 167.386 122.852) (width 0.25) (layer F.Cu) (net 1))
 (segment (start 166.54 113.284) (end 166.314999 113.509001) (width 0.25) (layer F.Cu) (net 1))
 (segment (start 167.64 113.284) (end 166.54 113.284) (width 0.4) (layer F.Cu) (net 1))
 (segment (start 171.45 101.854) (end 173.228 103.632) (width 0.4) (layer F.Cu) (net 1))
 (segment (start 168.03602 125.70202) (end 167.386 125.052) (width 0.25) (layer F.Cu) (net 1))
 (segment (start 178.84398 125.70202) (end 168.03602 125.70202) (width 0.25) (layer F.Cu) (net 1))
 (segment (start 167.386 125.052) (end 167.386 123.952) (width 0.25) (layer F.Cu) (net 1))
 (segment (start 180.594 123.952) (end 178.84398 125.70202) (width 0.25) (layer F.Cu) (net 1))
 (segment (start 193.2 100.1) (end 176.7 100.1) (width 0.4) (layer F.Cu) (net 1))
 (segment (start 176.7 100.1) (end 173.2 103.6) (width 0.4) (layer F.Cu) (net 1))
 (segment (start 183.3 106) (end 181.9 104.6) (width 0.25) (layer F.Cu) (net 1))
 (segment (start 181.9 104.6) (end 181.1 104.6) (width 0.25) (layer F.Cu) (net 1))
 (segment (start 179.3 105.05) (end 179.75 104.6) (width 0.25) (layer F.Cu) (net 1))
 (segment (start 178.6 105.05) (end 179.3 105.05) (width 0.25) (layer F.Cu) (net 1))
 (segment (start 179.75 104.6) (end 181 104.6) (width 0.25) (layer F.Cu) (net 1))
 (segment (start 190.6 107) (end 191 107.4) (width 0.4) (layer F.Cu) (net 1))
 (segment (start 189.55 107) (end 190.6 107) (width 0.4) (layer F.Cu) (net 1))
 (segment (start 191.001 107.399) (end 191 107.4) (width 0.25) (layer F.Cu) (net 1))
 (segment (start 192.786 107.399) (end 191.001 107.399) (width 0.4) (layer F.Cu) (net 1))
 (segment (start 183.3 106) (end 184.3 107) (width 0.25) (layer F.Cu) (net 1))
 (segment (start 184.3 107) (end 189.6 107) (width 0.25) (layer F.Cu) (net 1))
 (segment (start 193.2 100.1) (end 195.825001 102.725001) (width 0.4) (layer F.Cu) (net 1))
 (segment (start 195.825001 102.725001) (end 195.825001 105.048001) (width 0.4) (layer F.Cu) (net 1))
 (segment (start 195.8 105.073002) (end 195.825001 105.048001) (width 0.25) (layer F.Cu) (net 1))
 (segment (start 195.8 105.085) (end 195.8 105.073002) (width 0.25) (layer F.Cu) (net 1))
 (segment (start 193.486 107.399) (end 195.8 105.085) (width 0.4) (layer F.Cu) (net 1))
 (segment (start 192.786 107.399) (end 193.486 107.399) (width 0.25) (layer F.Cu) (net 1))
 (segment (start 212.575 100.1) (end 215.9 103.425) (width 0.4) (layer F.Cu) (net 1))
 (segment (start 193.2 100.1) (end 212.575 100.1) (width 0.4) (layer F.Cu) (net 1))
 (segment (start 215.9 103.425) (end 216.925 103.425) (width 0.4) (layer F.Cu) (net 1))
 (segment (start 171.45 96.472792) (end 171.45 101.854) (width 0.4) (layer F.Cu) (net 1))
 (segment (start 170.25 95.272792) (end 171.45 96.472792) (width 0.4) (layer F.Cu) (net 1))
 (segment (start 170.25 94) (end 170.25 95.272792) (width 0.4) (layer F.Cu) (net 1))
 (segment (start 165.75 112.494) (end 166.54 113.284) (width 0.4) (layer F.Cu) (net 1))
 (segment (start 166.878 101.854) (end 166.314999 102.417001) (width 0.4) (layer F.Cu) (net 1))
 (segment (start 171.45 101.854) (end 166.878 101.854) (width 0.4) (layer F.Cu) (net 1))
 (segment (start 166.314999 102.417001) (end 166.314999 102.435001) (width 0.4) (layer F.Cu) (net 1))
 (segment (start 166.314999 102.435001) (end 165.75 103) (width 0.4) (layer F.Cu) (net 1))
 (segment (start 165.75 103) (end 165.75 112.494) (width 0.4) (layer F.Cu) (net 1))
 (segment (start 181.05 108.6) (end 179.1 108.6) (width 0.25) (layer F.Cu) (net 17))
 (segment (start 179.1 108.6) (end 171.5 116.2) (width 0.25) (layer F.Cu) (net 17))
 (segment (start 181.975 110.85) (end 173.125 119.7) (width 0.25) (layer F.Cu) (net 16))
 (segment (start 182.5 110.85) (end 181.975 110.85) (width 0.25) (layer F.Cu) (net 16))
 (segment (start 173.125 119.7) (end 171.4 119.7) (width 0.25) (layer F.Cu) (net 16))
 (via (at 178.7 110.2) (size 0.8) (drill 0.4) (layers F.Cu B.Cu) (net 2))
 (segment (start 181.05 109.4) (end 179.5 109.4) (width 0.25) (layer F.Cu) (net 2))
 (segment (start 179.5 109.4) (end 178.7 110.2) (width 0.25) (layer F.Cu) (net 2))
 (segment (start 178.7 110.2) (end 175.7 107.2) (width 0.25) (layer B.Cu) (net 2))
 (via (at 174.75 100.75) (size 0.8) (drill 0.4) (layers F.Cu B.Cu) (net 2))
 (segment (start 175.7 107.2) (end 175.7 101.7) (width 0.25) (layer B.Cu) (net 2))
 (segment (start 175.7 101.7) (end 174.75 100.75) (width 0.25) (layer B.Cu) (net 2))
 (segment (start 172.75 98.75) (end 172.75 94) (width 0.25) (layer F.Cu) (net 2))
 (segment (start 174.75 100.75) (end 172.75 98.75) (width 0.25) (layer F.Cu) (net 2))
 (via (at 186.5 107.8) (size 0.8) (drill 0.4) (layers F.Cu B.Cu) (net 13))
 (segment (start 186.5 110.85) (end 186.5 107.8) (width 0.25) (layer F.Cu) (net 13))
 (segment (start 186.5 107.8) (end 186.5 117.8) (width 0.25) (layer B.Cu) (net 13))
 (segment (start 186.5 117.8) (end 183.1 121.2) (width 0.25) (layer B.Cu) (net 13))
 (segment (start 183.1 121.2) (end 183.1 124) (width 0.25) (layer B.Cu) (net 13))
 (segment (start 187.3 117.63641) (end 187.3 108.5) (width 0.25) (layer B.Cu) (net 12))
 (segment (start 184.404 123.952) (end 184.404 120.53241) (width 0.25) (layer B.Cu) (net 12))
 (via (at 187.3 108.5) (size 0.8) (drill 0.4) (layers F.Cu B.Cu) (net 12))
 (segment (start 184.404 120.53241) (end 187.3 117.63641) (width 0.25) (layer B.Cu) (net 12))
 (segment (start 187.3 108.5) (end 187.3 110.8) (width 0.25) (layer F.Cu) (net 12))
 (via (at 188.1 109.2) (size 0.8) (drill 0.4) (layers F.Cu B.Cu) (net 11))
 (segment (start 188.1 110.85) (end 188.1 109.2) (width 0.25) (layer F.Cu) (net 11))
 (segment (start 188.1 109.2) (end 188.1 118.1) (width 0.25) (layer B.Cu) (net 11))
 (segment (start 188.1 118.1) (end 185.7 120.5) (width 0.25) (layer B.Cu) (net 11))
 (segment (start 185.7 120.5) (end 185.7 124) (width 0.25) (layer B.Cu) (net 11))
 (segment (start 184.9 110.85) (end 184.9 111.873592) (width 0.25) (layer F.Cu) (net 10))
 (segment (start 184.9 111.873592) (end 185.626408 112.6) (width 0.25) (layer F.Cu) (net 10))
 (segment (start 185.626408 112.6) (end 195.86359 112.6) (width 0.25) (layer F.Cu) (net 10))
 (segment (start 212.724989 105.324989) (end 215.225001 107.825001) (width 0.25) (layer F.Cu) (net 10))
 (segment (start 195.86359 112.6) (end 203.138601 105.324989) (width 0.25) (layer F.Cu) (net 10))
 (segment (start 203.138601 105.324989) (end 212.724989 105.324989) (width 0.25) (layer F.Cu) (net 10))
 (segment (start 215.225001 107.825001) (end 215.9 108.5) (width 0.25) (layer F.Cu) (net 10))
 (segment (start 215.9 108.5) (end 216.9 108.5) (width 0.25) (layer F.Cu) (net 10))
 (segment (start 216.9 108.5) (end 217 108.6) (width 0.25) (layer F.Cu) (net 10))
 (segment (start 185.489998 113.1) (end 184.1 111.710002) (width 0.25) (layer F.Cu) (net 9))
 (segment (start 196 113.1) (end 185.489998 113.1) (width 0.25) (layer F.Cu) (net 9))
 (segment (start 184.1 111.710002) (end 184.1 111) (width 0.25) (layer F.Cu) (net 9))
 (segment (start 203.325001 105.774999) (end 208.874999 105.774999) (width 0.25) (layer F.Cu) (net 9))
 (segment (start 196 113.1) (end 203.325001 105.774999) (width 0.25) (layer F.Cu) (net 9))
 (segment (start 208.874999 105.774999) (end 213.6 110.5) (width 0.25) (layer F.Cu) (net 9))
 (segment (start 215.7 110.5) (end 216.3 110.5) (width 0.25) (layer F.Cu) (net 9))
 (segment (start 215.7 110.5) (end 215.9 110.5) (width 0.25) (layer F.Cu) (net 9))
 (segment (start 213.6 110.5) (end 215.7 110.5) (width 0.25) (layer F.Cu) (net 9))
 (segment (start 216.3 110.5) (end 217 111.2) (width 0.25) (layer F.Cu) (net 9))
 (segment (start 199.8 112.85) (end 200.75 111.9) (width 0.4) (layer F.Cu) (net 7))
 (segment (start 199.8 114) (end 199.8 112.85) (width 0.4) (layer F.Cu) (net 7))
 (segment (start 200.75 111.9) (end 202.1 111.9) (width 0.4) (layer F.Cu) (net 7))
 (segment (start 202.1 111.9) (end 204.7 114.5) (width 0.4) (layer F.Cu) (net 7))
 (segment (start 187.34999 113.55001) (end 196.186401 113.550009) (width 0.25) (layer F.Cu) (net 8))
 (segment (start 196.186401 113.550009) (end 201.668205 108.068205) (width 0.25) (layer F.Cu) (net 8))
 (segment (start 207.081795 108.068205) (end 207.2 107.95) (width 0.25) (layer F.Cu) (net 8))
 (segment (start 201.668205 108.068205) (end 207.081795 108.068205) (width 0.25) (layer F.Cu) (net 8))
 (segment (start 207.2 107.95) (end 207.2 106.9) (width 0.25) (layer F.Cu) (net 8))
 (segment (start 187.19999 113.55001) (end 187.34999 113.55001) (width 0.25) (layer F.Cu) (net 8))
 (segment (start 184.545 116.205) (end 187.19999 113.55001) (width 0.25) (layer F.Cu) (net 8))
 (segment (start 179.07 116.205) (end 184.545 116.205) (width 0.25) (layer F.Cu) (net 8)))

